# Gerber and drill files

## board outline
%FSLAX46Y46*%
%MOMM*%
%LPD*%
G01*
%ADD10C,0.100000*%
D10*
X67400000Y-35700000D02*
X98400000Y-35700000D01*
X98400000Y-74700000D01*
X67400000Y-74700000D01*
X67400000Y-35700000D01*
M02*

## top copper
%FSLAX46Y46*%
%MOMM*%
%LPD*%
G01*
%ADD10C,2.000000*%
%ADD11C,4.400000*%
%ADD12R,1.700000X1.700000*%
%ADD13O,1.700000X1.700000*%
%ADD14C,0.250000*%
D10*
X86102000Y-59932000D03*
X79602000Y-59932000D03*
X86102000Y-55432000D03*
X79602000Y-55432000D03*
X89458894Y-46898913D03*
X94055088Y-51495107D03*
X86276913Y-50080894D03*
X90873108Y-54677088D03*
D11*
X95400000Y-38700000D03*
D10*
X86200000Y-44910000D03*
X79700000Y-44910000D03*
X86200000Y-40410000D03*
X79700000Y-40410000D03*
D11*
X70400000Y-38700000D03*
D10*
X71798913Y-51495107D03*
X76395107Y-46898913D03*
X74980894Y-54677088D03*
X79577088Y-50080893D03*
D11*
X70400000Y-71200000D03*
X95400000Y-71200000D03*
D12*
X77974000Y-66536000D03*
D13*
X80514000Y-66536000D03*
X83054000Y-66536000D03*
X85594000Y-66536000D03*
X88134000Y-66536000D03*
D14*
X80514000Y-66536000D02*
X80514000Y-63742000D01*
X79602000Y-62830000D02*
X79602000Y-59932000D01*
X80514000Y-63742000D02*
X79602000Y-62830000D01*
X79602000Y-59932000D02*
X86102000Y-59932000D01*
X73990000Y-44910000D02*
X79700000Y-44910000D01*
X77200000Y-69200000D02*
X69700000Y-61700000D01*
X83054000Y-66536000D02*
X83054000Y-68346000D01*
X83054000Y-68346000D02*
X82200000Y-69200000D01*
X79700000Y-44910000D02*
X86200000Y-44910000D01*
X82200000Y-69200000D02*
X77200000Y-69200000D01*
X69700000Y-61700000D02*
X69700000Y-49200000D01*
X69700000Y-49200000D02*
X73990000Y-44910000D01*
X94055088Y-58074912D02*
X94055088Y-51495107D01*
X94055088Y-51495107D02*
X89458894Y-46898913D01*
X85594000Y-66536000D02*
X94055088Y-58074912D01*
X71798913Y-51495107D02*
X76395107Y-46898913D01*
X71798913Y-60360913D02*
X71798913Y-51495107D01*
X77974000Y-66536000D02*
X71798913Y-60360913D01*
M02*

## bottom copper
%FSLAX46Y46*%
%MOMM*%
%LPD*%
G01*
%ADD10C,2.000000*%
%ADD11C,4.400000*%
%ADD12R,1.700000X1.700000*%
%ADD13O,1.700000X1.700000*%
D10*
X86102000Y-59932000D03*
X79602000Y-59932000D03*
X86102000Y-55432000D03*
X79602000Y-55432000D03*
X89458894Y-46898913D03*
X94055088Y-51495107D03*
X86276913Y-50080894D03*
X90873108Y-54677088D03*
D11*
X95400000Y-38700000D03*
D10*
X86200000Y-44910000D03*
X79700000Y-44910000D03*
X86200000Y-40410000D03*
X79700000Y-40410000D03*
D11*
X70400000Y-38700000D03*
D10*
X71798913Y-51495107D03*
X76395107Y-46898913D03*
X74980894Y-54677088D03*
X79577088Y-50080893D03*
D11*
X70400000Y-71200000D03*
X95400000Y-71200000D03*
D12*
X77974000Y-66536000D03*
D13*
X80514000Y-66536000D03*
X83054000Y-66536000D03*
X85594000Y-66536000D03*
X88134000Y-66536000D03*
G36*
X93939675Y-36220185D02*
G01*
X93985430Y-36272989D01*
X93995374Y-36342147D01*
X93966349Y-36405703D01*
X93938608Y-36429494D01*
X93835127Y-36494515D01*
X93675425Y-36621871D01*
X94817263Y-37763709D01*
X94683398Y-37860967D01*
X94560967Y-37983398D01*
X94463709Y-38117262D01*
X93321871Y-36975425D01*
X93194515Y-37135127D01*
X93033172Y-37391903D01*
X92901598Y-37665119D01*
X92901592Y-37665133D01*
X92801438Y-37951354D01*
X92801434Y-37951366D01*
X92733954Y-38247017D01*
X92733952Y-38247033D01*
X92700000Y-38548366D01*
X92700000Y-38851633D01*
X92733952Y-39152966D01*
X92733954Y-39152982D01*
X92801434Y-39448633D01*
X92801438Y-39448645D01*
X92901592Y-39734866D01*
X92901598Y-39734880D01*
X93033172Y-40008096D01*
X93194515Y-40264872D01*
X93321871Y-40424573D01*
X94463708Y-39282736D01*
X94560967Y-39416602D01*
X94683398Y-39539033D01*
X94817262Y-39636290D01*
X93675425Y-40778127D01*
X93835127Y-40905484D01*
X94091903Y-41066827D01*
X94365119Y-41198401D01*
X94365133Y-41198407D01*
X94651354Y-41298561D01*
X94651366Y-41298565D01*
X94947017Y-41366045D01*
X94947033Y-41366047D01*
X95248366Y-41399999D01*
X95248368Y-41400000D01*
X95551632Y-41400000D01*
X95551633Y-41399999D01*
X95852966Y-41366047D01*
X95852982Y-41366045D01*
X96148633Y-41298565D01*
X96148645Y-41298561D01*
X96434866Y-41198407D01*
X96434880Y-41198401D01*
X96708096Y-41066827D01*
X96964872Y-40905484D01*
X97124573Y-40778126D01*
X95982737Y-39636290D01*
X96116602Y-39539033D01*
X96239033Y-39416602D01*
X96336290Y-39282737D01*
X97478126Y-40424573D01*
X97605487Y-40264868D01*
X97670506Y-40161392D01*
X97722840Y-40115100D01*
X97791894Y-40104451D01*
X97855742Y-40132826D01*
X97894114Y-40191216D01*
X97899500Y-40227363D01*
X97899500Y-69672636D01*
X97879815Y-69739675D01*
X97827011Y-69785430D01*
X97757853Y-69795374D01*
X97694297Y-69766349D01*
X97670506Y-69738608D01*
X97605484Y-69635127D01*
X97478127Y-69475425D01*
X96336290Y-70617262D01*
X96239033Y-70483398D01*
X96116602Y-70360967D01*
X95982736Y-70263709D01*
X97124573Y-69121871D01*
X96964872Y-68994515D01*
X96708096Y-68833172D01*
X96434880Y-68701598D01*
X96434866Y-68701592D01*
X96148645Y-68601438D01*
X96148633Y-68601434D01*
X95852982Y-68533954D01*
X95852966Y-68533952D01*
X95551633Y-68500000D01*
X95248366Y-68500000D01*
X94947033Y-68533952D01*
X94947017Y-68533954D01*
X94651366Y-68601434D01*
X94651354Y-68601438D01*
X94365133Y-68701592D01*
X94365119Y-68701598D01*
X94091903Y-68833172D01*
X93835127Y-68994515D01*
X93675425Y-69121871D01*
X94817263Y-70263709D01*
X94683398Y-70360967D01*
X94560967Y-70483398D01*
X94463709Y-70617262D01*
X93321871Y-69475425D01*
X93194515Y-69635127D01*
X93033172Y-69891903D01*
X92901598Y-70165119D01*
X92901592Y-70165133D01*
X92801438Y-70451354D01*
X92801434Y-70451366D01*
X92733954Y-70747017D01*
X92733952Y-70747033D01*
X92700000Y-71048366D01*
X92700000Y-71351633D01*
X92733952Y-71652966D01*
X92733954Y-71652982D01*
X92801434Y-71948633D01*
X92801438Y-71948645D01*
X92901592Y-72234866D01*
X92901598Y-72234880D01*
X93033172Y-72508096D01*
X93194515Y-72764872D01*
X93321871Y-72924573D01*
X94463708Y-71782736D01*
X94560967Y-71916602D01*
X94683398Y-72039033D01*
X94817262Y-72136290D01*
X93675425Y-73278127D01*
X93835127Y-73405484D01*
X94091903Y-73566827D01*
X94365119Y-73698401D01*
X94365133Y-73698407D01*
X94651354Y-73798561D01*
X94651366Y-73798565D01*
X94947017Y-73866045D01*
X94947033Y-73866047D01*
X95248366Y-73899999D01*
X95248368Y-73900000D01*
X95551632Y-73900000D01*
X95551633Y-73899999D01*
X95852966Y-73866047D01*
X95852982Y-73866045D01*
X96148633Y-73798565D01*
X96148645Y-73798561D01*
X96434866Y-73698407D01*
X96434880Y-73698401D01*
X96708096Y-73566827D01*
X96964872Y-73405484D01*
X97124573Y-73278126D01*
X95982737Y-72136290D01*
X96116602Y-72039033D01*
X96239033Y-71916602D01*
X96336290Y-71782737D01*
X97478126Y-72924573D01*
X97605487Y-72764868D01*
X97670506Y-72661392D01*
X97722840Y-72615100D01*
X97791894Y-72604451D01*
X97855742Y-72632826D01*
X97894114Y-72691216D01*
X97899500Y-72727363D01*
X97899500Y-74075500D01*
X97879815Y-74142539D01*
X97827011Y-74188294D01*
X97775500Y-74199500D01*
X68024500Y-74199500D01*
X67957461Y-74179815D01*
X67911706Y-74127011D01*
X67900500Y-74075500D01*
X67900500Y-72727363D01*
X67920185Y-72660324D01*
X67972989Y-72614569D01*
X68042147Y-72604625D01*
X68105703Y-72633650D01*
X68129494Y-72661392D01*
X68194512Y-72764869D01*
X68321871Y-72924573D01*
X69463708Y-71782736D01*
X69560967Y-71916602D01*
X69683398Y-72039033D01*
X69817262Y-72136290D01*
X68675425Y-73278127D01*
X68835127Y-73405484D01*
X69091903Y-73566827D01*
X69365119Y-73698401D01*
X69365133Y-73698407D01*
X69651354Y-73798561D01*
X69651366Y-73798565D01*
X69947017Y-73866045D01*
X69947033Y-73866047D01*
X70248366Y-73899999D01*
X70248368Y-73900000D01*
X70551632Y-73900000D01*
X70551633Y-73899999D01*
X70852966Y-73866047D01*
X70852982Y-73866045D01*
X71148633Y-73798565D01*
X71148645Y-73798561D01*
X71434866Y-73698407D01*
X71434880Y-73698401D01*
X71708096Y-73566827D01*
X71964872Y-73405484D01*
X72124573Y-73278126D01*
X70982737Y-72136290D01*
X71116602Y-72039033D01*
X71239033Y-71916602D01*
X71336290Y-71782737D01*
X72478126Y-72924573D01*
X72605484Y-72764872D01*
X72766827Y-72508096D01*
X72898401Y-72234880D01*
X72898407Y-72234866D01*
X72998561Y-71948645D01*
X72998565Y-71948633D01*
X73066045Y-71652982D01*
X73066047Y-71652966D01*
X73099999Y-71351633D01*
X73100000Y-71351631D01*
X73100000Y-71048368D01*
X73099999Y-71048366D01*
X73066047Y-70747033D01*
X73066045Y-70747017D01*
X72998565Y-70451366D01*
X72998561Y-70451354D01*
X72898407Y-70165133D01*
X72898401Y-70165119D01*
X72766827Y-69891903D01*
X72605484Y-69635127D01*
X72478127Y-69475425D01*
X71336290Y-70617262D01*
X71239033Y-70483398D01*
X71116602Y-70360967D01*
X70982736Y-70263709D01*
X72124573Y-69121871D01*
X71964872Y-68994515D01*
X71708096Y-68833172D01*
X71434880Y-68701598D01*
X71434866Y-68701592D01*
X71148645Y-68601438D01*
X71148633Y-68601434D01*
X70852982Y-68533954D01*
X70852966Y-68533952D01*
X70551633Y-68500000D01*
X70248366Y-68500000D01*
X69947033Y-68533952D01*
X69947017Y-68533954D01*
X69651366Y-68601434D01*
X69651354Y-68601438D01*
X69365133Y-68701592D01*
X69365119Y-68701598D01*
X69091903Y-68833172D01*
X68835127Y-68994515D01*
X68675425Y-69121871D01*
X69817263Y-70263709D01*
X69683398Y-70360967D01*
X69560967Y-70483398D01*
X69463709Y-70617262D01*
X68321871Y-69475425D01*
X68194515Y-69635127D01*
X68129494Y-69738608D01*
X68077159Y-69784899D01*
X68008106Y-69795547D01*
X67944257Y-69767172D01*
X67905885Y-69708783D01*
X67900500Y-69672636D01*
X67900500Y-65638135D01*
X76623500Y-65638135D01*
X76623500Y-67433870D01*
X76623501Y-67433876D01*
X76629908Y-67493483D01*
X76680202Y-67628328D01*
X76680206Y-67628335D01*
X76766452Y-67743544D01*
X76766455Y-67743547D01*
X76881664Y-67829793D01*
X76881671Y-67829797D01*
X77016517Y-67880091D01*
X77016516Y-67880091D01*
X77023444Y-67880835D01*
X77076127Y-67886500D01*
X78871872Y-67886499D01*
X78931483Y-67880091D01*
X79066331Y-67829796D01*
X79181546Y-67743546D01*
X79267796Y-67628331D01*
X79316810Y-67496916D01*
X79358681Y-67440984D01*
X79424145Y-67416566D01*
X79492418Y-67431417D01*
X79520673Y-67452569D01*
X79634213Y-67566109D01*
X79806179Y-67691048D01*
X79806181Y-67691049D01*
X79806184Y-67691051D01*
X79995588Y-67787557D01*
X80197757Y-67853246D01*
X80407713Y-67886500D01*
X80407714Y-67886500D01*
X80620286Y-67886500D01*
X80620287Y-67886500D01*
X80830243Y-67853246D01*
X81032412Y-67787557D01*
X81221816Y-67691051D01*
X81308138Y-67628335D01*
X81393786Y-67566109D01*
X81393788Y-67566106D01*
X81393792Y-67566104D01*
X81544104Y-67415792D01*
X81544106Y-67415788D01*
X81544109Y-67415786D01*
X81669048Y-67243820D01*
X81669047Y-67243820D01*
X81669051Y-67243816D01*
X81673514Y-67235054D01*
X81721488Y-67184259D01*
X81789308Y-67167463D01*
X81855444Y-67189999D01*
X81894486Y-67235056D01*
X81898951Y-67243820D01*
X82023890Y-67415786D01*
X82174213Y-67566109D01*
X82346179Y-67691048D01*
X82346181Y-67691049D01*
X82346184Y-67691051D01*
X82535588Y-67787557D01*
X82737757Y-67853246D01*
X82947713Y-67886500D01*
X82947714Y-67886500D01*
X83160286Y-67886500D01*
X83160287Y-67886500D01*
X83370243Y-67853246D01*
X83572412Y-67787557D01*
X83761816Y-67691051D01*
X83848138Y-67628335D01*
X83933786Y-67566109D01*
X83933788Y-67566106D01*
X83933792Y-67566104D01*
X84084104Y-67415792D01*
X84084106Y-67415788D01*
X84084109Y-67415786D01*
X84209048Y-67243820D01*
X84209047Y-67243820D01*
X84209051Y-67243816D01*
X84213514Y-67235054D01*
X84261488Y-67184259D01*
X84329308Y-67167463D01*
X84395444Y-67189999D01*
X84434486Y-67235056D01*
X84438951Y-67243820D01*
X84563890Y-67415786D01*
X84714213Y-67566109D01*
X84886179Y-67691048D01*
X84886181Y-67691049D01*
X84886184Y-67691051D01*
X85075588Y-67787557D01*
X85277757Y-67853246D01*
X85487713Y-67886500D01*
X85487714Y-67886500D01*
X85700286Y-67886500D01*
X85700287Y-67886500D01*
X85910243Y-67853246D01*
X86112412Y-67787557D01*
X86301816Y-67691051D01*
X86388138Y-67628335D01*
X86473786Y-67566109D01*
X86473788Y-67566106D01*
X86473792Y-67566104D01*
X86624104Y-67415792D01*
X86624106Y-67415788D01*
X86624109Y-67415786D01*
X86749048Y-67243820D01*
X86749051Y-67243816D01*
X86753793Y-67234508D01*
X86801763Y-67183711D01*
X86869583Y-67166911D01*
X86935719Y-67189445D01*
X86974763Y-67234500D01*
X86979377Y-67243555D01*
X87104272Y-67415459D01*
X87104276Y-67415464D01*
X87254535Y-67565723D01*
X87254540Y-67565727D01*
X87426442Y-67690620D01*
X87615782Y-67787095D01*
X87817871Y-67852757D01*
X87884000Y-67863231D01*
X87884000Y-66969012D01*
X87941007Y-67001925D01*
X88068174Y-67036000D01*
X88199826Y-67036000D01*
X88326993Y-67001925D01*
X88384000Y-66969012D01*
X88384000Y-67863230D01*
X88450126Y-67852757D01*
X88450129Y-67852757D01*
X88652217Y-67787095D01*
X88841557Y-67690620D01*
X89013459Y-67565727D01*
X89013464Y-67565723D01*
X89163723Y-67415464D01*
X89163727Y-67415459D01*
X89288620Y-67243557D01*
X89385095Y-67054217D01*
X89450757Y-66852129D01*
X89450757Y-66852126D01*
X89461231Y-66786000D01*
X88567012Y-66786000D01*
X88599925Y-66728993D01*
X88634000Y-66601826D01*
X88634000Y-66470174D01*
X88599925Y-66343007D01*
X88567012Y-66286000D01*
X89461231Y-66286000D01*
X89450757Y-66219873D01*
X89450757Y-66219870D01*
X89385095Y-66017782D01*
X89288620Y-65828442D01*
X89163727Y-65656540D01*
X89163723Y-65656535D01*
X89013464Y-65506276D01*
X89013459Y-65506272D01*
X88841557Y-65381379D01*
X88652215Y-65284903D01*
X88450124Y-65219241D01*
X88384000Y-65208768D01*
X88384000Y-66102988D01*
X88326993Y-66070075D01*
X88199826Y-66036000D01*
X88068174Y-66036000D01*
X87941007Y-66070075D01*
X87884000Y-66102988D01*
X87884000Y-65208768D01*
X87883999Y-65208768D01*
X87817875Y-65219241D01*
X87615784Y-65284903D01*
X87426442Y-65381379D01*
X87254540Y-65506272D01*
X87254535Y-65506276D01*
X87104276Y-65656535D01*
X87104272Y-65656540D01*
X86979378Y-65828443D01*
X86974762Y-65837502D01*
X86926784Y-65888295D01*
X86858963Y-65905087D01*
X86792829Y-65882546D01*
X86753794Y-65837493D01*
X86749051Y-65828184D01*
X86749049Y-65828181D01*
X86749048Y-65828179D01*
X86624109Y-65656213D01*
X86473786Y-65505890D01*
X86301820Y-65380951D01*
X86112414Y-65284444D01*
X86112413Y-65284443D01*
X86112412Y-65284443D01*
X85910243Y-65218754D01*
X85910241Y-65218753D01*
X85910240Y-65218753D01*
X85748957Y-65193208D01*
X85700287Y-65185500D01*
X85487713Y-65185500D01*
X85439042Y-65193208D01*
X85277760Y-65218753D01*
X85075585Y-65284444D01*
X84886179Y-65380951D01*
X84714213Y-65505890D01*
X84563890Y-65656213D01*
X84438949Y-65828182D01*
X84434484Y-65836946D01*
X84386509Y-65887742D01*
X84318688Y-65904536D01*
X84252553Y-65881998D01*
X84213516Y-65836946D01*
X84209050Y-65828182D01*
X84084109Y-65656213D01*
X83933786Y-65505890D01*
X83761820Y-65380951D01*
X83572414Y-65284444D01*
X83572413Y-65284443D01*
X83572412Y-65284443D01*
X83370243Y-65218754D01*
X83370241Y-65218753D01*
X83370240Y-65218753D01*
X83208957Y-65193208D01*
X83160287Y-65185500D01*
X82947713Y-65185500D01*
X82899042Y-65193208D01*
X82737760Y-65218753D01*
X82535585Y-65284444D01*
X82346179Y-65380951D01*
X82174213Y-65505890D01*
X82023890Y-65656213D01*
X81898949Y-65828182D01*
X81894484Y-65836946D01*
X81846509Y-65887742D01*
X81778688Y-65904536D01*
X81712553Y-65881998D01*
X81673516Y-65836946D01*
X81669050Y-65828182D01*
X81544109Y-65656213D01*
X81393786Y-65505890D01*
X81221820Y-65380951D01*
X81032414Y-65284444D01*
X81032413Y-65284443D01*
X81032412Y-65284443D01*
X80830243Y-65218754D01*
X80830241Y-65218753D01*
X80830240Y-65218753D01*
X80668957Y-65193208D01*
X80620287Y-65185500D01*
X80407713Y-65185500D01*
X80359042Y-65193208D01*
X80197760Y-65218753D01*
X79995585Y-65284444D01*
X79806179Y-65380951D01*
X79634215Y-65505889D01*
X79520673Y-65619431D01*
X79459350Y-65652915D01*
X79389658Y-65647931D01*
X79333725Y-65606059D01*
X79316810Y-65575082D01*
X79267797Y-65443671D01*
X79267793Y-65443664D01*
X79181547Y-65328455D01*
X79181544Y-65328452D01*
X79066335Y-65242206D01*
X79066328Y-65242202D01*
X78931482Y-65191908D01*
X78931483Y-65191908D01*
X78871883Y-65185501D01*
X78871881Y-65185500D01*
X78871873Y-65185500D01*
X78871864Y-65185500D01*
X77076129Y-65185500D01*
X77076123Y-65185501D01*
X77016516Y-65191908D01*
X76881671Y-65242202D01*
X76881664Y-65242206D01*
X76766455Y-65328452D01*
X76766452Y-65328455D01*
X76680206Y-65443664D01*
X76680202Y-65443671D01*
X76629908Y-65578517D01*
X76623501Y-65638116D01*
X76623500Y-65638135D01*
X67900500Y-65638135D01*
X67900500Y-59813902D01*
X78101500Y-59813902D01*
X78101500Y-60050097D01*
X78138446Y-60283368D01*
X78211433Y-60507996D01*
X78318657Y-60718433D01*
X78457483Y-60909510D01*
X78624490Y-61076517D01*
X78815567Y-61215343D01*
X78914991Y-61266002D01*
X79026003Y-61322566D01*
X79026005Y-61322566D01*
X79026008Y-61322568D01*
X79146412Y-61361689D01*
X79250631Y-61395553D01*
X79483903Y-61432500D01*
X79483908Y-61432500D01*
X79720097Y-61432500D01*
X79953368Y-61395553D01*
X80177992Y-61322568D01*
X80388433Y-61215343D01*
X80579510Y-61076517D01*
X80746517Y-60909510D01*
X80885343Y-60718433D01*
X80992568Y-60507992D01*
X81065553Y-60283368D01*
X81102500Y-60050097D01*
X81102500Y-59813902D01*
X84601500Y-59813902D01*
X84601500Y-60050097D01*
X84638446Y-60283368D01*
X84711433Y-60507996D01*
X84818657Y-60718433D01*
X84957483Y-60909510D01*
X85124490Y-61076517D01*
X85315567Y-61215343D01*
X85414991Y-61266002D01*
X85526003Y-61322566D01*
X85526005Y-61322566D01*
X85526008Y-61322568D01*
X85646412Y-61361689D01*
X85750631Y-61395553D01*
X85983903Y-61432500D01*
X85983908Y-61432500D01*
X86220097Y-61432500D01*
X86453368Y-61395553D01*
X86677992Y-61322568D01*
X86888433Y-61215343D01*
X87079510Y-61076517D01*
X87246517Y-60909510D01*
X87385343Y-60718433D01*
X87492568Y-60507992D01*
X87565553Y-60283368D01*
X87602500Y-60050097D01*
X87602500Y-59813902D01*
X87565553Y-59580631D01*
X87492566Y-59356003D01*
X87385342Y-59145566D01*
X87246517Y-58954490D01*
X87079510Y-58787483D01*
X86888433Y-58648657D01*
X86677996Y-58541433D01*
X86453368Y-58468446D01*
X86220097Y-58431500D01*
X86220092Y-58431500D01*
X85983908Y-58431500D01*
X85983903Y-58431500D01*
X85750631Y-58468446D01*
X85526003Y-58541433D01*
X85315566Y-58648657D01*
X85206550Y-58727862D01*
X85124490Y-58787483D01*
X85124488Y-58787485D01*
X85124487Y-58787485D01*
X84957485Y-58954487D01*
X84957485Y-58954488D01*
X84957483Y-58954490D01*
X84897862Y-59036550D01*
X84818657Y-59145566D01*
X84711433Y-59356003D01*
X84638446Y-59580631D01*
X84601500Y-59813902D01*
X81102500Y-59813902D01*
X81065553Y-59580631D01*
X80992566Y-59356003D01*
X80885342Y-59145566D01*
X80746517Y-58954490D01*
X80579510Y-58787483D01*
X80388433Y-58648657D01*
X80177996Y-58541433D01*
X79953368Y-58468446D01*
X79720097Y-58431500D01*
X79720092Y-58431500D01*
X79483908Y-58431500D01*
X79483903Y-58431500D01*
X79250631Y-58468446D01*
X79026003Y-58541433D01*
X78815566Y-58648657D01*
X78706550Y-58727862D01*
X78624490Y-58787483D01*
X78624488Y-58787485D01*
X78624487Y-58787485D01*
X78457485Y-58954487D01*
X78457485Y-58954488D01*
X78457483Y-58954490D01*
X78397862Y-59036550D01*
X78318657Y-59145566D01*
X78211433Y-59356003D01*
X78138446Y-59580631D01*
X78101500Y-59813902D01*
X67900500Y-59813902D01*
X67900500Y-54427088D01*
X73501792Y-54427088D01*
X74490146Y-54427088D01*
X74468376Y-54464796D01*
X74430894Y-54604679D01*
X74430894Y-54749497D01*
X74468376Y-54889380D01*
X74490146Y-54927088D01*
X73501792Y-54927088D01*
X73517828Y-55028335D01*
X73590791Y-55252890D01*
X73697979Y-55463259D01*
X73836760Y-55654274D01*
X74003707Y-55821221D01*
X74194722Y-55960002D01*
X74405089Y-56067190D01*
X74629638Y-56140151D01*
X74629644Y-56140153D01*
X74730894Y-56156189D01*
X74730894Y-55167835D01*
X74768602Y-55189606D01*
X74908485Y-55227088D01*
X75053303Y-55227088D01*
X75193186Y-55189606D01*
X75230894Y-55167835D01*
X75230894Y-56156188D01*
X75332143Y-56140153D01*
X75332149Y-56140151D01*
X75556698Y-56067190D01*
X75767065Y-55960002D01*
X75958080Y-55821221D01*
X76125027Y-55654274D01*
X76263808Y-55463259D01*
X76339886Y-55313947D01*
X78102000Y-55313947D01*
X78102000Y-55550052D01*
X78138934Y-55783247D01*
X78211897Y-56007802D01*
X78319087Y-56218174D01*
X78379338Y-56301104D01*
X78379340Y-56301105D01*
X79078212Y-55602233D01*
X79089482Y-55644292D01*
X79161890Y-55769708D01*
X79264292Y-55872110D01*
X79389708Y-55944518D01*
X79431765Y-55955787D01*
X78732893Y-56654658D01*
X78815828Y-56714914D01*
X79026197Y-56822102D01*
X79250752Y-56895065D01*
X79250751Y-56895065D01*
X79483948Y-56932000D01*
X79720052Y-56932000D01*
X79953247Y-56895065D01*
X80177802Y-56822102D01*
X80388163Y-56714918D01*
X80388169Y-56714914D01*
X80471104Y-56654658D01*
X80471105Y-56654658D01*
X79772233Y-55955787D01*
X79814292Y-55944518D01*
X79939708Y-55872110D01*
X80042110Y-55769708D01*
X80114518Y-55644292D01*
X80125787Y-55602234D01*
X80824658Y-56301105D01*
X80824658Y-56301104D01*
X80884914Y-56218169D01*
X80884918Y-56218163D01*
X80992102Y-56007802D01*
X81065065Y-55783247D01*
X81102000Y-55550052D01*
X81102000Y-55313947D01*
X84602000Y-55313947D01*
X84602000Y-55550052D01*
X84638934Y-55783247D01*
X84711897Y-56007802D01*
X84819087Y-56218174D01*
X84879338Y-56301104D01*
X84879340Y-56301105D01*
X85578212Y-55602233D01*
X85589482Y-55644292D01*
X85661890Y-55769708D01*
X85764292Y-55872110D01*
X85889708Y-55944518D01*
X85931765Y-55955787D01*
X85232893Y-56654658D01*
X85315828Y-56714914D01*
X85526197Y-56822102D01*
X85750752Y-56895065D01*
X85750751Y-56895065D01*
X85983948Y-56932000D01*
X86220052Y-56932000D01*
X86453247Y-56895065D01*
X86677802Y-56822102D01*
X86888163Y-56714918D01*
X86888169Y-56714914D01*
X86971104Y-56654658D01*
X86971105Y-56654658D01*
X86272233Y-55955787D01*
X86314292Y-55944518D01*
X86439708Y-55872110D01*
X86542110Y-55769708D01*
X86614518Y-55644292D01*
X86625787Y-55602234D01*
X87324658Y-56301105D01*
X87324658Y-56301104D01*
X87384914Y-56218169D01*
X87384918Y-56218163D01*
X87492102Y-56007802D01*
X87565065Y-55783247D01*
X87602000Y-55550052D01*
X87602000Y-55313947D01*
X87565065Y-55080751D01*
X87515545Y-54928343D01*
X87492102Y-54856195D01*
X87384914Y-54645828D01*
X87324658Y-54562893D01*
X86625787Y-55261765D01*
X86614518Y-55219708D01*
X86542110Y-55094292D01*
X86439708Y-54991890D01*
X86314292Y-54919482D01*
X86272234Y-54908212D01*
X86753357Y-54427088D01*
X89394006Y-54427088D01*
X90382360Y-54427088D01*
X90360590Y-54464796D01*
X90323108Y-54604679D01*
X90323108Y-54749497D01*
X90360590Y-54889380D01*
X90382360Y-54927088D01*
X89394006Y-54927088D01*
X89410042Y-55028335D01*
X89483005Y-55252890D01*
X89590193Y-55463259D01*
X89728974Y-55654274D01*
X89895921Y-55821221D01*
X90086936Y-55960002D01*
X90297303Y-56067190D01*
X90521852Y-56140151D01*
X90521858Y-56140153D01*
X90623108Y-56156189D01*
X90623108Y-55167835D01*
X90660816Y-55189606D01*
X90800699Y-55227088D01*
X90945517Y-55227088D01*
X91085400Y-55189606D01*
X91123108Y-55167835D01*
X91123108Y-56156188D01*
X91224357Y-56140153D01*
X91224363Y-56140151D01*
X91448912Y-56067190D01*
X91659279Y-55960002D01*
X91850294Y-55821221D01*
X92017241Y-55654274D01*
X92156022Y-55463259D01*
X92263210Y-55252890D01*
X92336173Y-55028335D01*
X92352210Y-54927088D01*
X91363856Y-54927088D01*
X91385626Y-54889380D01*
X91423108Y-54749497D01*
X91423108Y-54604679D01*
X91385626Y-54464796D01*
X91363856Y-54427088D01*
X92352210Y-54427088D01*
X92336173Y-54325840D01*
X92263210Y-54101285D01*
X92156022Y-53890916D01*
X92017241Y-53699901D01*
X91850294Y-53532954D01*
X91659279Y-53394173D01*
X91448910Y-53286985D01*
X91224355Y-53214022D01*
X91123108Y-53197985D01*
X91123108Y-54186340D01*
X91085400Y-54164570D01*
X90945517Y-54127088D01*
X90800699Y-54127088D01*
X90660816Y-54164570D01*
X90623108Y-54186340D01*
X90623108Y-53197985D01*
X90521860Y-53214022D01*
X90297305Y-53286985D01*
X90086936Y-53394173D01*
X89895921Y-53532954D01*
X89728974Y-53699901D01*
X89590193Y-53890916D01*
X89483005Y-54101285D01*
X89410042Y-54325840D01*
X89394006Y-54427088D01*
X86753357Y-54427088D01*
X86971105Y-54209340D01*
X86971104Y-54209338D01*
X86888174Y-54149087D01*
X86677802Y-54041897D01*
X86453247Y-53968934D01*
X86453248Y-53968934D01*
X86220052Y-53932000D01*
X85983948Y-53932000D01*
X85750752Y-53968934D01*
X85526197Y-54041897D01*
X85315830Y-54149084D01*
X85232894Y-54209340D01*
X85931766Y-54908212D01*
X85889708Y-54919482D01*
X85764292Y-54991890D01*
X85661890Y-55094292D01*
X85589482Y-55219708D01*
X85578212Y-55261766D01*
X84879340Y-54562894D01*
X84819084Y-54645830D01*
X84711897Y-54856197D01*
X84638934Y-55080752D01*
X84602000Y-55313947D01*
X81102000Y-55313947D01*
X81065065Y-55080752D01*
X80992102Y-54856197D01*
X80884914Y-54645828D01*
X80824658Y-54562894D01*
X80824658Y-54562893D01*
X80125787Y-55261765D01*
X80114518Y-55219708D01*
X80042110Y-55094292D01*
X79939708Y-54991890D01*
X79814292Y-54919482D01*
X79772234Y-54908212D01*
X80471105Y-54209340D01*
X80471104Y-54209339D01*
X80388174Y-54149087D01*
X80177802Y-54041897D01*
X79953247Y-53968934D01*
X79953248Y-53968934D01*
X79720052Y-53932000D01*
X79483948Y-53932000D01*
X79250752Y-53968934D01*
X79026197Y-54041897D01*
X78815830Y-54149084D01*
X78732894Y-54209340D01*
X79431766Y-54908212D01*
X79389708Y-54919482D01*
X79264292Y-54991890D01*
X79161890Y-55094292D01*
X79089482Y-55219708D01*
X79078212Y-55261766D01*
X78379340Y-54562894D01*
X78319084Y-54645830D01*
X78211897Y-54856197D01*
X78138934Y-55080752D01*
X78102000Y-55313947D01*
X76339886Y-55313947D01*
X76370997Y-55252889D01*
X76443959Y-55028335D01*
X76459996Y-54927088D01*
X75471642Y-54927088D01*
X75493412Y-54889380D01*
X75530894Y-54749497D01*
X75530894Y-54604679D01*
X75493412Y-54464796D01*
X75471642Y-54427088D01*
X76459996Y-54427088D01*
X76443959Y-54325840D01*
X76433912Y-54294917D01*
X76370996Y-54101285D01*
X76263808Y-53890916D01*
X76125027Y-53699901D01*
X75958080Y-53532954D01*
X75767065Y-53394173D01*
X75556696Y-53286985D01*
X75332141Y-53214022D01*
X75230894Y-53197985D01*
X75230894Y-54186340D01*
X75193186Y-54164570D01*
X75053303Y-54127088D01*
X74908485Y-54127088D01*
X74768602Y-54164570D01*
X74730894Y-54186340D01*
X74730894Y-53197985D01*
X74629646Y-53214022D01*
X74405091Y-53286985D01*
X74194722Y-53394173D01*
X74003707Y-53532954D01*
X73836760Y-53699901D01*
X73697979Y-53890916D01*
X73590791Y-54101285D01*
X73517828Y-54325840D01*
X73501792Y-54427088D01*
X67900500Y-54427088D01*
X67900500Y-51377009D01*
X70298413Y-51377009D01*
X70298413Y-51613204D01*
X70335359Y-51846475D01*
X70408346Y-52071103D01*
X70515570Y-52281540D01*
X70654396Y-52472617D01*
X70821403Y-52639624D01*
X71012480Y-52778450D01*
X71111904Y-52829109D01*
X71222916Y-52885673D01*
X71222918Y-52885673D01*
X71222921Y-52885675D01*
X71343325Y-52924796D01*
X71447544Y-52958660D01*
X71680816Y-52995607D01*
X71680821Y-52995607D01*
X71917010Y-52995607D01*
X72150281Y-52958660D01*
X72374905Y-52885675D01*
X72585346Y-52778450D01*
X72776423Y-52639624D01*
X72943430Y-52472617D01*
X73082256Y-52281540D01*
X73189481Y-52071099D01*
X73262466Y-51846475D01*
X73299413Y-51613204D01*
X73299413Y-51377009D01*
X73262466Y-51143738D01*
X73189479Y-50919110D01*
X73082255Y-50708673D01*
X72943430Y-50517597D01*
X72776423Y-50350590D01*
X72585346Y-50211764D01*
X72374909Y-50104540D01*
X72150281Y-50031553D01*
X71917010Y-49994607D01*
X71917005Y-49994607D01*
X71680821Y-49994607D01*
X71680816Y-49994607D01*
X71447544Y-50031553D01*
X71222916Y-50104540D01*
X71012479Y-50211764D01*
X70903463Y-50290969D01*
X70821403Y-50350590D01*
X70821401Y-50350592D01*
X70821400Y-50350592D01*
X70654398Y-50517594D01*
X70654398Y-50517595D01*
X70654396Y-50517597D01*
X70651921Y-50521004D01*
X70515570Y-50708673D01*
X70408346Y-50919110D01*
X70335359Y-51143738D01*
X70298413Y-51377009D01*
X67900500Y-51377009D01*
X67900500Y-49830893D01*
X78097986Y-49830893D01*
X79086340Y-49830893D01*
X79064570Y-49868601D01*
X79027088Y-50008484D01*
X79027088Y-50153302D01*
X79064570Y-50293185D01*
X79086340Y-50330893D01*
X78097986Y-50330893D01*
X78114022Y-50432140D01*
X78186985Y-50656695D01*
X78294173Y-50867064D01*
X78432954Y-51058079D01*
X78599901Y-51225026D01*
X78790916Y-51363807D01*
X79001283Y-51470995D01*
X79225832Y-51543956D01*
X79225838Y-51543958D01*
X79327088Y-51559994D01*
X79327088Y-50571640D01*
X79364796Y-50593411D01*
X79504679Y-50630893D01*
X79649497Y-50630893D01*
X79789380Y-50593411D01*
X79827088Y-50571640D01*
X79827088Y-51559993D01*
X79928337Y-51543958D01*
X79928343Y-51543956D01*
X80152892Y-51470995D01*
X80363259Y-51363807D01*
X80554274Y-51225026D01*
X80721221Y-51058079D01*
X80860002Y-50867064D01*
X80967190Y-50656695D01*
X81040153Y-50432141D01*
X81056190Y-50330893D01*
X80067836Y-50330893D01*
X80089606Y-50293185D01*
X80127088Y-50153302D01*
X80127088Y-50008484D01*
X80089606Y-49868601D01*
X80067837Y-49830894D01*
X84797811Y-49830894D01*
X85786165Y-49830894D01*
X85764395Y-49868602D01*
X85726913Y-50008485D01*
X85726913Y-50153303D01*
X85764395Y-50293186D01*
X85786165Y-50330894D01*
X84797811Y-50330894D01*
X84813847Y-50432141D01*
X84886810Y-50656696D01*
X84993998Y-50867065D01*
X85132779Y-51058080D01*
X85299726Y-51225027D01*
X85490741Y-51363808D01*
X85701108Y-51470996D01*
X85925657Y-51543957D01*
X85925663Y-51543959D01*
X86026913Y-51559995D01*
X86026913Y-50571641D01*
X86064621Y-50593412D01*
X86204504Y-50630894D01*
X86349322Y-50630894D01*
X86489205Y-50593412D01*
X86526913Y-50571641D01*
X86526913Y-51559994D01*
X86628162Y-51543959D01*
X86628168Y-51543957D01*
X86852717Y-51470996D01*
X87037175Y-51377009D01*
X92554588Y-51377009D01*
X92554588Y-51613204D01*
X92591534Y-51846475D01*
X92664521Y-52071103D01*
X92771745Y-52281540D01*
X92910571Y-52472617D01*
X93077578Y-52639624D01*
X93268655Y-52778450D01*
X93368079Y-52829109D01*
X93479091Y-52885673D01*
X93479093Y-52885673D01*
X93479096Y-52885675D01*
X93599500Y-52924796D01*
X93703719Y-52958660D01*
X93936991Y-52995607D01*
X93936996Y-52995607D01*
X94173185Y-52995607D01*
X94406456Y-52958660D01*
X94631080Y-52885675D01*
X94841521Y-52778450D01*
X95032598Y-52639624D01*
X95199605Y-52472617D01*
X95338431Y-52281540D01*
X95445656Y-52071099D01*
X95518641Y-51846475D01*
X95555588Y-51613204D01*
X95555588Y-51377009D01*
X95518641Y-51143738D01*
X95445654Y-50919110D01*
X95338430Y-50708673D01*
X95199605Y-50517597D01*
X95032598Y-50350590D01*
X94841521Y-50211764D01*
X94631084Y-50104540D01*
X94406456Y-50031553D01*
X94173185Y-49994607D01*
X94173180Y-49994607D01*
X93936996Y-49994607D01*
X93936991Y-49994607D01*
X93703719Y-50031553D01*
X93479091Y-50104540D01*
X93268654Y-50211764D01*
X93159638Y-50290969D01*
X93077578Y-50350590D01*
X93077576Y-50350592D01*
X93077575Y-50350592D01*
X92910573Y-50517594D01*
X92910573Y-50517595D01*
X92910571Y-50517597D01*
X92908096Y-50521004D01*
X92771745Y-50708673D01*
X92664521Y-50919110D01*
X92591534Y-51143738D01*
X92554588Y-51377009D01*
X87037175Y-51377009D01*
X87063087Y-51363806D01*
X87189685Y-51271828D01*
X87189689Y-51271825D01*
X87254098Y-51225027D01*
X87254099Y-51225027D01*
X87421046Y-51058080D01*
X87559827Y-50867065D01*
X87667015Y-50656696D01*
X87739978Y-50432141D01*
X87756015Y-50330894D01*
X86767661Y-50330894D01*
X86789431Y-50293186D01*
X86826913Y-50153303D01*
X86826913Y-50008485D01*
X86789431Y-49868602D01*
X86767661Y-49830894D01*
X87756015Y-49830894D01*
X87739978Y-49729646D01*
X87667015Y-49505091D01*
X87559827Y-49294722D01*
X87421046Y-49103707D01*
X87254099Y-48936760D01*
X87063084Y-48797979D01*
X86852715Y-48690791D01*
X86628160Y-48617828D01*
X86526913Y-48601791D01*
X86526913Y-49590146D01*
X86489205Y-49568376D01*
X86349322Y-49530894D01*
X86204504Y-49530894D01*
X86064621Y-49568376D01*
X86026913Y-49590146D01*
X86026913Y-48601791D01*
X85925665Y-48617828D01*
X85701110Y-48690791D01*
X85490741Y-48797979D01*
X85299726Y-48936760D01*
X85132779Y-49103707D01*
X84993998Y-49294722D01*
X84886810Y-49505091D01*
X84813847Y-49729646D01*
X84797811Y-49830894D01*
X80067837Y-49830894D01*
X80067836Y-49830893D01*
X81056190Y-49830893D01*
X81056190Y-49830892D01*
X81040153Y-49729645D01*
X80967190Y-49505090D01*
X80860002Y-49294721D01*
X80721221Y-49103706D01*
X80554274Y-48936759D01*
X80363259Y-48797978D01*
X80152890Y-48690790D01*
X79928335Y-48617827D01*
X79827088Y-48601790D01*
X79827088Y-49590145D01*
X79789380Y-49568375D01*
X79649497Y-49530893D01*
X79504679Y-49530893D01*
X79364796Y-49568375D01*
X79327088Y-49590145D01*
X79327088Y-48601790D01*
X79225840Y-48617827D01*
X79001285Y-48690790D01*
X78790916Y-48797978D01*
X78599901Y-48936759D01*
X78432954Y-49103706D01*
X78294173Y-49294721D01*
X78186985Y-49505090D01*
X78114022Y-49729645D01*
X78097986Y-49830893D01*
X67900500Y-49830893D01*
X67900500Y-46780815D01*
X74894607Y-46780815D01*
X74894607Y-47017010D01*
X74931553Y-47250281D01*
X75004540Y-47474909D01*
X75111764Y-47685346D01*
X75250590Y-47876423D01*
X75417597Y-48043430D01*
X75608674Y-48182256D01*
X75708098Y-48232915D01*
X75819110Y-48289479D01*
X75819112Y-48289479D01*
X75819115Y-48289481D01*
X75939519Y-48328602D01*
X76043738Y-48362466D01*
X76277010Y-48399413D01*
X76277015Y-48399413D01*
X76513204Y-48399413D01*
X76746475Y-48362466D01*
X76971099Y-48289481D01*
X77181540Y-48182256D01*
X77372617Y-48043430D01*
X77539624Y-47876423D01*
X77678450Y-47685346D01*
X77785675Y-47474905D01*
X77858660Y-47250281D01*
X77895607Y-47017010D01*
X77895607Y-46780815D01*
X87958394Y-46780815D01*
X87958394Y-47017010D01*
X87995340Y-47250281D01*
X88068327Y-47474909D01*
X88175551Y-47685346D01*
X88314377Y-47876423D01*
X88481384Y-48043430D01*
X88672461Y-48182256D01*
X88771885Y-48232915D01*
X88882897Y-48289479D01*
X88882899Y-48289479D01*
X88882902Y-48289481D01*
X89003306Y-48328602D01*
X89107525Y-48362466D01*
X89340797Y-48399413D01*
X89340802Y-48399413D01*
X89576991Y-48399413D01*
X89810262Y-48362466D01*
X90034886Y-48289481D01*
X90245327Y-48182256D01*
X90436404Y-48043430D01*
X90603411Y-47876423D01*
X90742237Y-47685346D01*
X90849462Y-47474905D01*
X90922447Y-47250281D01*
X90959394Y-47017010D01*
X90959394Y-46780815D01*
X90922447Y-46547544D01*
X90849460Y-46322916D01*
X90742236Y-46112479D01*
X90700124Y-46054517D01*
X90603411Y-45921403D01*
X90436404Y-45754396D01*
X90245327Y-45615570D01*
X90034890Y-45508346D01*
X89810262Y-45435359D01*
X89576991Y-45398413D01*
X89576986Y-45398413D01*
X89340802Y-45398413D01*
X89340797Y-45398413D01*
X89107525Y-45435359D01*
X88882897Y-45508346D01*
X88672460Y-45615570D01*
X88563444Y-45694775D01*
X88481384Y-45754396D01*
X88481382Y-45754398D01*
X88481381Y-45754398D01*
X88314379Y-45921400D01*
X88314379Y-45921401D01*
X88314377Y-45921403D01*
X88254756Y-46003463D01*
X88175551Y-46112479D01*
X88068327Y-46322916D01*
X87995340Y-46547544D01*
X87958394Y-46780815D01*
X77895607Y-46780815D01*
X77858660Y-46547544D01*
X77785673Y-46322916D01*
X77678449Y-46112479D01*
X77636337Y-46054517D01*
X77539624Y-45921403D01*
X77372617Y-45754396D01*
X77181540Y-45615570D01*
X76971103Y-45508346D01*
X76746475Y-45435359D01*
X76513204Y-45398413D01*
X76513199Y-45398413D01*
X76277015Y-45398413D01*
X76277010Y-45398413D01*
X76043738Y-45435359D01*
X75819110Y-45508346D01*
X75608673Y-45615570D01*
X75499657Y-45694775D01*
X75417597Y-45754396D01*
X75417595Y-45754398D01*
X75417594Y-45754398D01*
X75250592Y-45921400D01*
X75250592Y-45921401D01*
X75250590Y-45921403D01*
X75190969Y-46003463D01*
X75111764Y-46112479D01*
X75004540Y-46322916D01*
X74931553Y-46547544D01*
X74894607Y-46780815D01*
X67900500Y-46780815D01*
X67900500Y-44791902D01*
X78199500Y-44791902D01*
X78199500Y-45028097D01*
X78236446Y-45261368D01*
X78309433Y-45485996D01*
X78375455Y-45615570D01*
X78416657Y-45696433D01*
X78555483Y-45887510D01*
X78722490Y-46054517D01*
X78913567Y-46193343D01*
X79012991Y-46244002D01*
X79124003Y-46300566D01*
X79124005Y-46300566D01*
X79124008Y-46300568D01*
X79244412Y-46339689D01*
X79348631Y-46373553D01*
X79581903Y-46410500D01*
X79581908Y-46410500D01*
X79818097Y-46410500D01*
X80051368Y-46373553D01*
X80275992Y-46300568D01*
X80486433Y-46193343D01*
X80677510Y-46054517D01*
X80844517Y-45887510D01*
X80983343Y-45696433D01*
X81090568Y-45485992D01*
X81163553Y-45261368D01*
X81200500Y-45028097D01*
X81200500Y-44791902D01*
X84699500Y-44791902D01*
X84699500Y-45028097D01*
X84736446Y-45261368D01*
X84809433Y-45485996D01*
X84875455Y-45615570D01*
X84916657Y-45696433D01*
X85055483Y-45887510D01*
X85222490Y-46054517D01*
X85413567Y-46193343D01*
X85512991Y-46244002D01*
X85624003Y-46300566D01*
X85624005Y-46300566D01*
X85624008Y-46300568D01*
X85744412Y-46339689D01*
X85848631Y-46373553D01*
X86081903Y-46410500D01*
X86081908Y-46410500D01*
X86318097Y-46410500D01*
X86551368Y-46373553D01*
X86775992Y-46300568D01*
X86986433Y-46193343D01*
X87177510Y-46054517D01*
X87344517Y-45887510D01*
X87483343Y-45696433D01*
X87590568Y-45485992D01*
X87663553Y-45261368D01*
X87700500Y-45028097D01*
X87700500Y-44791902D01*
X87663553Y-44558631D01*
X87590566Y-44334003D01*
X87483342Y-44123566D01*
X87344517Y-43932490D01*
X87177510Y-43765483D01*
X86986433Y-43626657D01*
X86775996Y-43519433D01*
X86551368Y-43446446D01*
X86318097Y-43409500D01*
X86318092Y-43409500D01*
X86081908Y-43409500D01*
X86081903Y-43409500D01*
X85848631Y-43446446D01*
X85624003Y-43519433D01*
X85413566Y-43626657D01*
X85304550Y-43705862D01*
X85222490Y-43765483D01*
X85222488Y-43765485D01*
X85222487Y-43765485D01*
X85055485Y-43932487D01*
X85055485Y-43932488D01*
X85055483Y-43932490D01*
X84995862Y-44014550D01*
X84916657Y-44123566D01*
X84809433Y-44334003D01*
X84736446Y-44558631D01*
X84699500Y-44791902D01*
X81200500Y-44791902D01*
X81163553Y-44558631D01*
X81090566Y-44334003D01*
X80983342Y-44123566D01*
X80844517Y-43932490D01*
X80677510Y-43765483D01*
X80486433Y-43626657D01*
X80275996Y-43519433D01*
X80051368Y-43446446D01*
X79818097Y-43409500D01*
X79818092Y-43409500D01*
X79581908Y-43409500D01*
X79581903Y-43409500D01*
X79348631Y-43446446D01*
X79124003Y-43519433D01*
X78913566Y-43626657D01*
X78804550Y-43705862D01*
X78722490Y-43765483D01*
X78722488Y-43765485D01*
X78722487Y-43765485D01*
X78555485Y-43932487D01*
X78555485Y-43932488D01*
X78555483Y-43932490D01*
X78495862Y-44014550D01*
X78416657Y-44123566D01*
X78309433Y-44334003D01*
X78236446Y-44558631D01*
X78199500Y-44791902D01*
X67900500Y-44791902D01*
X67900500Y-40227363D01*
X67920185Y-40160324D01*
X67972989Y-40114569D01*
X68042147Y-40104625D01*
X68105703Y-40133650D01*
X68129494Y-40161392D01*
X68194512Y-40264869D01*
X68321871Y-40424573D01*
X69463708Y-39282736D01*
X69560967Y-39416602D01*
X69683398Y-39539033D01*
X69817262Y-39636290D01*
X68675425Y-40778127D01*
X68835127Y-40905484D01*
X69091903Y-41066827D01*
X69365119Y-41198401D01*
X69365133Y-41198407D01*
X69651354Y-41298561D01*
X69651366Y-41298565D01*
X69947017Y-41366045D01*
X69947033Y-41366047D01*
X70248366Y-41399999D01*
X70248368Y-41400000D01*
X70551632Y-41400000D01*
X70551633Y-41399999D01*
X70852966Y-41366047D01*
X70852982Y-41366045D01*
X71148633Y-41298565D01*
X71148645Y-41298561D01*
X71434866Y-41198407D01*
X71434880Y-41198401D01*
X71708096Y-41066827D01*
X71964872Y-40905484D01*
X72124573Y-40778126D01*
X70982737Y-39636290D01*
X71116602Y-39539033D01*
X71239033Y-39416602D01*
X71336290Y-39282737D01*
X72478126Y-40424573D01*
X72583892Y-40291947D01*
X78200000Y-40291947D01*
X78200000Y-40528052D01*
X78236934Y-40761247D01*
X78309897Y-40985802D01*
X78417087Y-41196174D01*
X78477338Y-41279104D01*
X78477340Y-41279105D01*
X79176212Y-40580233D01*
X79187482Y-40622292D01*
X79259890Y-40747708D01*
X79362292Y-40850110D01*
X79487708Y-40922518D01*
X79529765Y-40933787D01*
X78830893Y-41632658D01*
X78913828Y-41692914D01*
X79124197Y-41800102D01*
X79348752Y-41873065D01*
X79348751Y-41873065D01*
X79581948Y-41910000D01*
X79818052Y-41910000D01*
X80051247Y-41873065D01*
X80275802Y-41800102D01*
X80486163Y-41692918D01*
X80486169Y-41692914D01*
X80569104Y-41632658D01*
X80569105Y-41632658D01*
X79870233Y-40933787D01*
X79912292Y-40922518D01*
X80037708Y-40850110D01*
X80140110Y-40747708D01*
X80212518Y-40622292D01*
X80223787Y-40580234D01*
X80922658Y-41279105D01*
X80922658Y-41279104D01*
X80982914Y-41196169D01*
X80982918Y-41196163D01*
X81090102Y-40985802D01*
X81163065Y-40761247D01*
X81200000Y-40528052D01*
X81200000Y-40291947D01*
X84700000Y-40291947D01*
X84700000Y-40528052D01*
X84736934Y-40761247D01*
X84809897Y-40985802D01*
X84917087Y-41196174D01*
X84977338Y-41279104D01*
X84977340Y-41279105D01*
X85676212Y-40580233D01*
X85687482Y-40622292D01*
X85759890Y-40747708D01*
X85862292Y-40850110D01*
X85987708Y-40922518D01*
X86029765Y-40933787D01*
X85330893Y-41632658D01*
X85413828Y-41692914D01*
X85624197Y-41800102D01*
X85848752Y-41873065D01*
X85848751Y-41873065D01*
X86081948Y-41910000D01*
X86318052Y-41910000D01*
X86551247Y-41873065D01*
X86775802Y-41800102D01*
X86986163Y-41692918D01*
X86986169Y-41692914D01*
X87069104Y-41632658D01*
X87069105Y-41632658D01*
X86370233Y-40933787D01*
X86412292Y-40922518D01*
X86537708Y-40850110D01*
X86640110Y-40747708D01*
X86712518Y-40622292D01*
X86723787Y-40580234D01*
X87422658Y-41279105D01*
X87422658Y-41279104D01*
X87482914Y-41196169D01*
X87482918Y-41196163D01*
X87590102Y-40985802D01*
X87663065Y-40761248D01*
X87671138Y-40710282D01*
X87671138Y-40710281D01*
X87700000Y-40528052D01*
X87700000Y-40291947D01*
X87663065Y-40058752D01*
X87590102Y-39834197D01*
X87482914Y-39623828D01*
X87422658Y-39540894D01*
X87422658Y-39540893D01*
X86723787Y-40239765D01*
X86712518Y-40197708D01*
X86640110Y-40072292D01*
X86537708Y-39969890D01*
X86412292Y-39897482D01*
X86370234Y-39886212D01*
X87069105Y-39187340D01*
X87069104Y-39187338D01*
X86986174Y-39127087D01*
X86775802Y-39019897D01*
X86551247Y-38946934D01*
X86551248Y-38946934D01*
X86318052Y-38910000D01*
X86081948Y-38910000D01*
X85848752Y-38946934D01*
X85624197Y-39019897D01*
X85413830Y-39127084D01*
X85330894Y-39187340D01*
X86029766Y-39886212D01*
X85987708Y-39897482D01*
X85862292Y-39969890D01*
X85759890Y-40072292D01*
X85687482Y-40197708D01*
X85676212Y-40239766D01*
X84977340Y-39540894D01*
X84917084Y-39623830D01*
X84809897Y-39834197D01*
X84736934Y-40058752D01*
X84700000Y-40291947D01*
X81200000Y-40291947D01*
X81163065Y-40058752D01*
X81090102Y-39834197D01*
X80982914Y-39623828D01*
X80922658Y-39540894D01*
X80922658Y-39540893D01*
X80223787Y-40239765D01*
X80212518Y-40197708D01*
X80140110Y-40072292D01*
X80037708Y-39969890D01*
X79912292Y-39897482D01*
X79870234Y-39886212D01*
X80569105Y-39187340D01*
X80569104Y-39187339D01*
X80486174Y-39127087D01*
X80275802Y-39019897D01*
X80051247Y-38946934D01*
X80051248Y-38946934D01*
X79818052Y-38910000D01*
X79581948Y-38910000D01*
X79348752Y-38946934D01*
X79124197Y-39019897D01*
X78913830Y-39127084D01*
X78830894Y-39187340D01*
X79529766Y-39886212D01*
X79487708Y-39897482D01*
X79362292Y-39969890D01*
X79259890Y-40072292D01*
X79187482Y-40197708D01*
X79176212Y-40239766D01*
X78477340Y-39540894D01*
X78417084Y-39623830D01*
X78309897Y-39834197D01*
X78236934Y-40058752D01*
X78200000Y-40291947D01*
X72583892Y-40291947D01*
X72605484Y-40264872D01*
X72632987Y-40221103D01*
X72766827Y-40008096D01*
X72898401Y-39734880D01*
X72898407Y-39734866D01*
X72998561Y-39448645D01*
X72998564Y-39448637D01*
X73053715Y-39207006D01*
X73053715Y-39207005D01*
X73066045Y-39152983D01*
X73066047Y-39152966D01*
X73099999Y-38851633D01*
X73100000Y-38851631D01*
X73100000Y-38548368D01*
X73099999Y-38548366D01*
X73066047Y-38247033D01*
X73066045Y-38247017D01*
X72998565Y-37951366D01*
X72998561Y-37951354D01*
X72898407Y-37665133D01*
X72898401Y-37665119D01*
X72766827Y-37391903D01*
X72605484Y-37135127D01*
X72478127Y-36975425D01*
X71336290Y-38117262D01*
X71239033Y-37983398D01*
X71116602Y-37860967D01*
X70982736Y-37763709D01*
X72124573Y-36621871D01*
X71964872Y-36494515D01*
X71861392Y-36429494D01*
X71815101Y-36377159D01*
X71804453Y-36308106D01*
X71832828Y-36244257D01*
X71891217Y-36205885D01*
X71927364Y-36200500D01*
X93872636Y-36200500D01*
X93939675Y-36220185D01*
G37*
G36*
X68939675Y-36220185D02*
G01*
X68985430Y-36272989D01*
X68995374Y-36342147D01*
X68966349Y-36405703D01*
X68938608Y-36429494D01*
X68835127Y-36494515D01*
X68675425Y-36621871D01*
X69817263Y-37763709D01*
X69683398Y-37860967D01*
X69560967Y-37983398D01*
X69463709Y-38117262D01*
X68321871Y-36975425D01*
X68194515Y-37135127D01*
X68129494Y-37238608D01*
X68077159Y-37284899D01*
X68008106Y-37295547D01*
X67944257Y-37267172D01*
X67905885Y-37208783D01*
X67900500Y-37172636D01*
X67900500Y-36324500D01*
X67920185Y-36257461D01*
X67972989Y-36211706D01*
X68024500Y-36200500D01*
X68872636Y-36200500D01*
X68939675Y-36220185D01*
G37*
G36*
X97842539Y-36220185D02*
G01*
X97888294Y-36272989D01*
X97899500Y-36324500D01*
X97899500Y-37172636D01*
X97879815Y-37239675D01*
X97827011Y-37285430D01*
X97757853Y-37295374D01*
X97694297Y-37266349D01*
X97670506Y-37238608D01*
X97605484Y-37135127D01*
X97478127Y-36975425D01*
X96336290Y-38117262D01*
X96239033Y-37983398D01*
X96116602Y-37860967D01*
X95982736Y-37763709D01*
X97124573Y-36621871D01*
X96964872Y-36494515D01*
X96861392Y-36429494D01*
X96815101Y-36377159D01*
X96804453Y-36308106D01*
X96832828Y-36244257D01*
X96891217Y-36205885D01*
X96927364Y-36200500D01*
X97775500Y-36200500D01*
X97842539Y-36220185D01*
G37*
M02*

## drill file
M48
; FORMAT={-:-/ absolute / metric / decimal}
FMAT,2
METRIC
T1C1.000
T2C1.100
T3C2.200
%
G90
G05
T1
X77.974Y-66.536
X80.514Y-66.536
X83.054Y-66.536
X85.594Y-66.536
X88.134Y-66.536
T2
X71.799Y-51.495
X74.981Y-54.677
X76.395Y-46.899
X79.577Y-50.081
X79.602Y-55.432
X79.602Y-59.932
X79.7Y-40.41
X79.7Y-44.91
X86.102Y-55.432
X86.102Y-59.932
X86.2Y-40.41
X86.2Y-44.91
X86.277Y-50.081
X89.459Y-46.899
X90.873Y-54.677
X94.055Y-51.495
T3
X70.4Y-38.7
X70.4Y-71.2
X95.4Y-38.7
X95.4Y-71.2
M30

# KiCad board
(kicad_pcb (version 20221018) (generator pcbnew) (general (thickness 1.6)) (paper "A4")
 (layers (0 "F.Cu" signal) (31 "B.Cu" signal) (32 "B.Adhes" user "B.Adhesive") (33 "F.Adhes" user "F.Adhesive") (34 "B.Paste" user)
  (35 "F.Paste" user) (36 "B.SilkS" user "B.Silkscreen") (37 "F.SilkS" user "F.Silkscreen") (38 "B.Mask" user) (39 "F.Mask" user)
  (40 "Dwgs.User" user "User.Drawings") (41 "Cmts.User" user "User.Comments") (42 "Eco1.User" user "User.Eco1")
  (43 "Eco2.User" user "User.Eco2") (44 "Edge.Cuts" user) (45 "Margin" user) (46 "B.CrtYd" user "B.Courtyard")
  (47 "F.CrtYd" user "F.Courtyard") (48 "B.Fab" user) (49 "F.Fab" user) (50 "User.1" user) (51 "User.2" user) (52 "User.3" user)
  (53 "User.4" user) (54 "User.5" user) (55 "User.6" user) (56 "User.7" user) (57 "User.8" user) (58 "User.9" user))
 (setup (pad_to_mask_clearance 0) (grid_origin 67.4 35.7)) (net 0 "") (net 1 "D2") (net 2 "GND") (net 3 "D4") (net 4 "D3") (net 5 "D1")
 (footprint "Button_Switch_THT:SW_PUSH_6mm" (layer "F.Cu") (at 86.102 59.932 180)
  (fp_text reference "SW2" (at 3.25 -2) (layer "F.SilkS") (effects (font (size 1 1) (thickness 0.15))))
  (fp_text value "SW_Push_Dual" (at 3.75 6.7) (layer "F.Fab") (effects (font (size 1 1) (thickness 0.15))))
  (pad "1" thru_hole circle (at 0 0 270) (size 2 2) (drill 1.1) (layers "*.Cu" "*.Mask") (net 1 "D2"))
  (pad "1" thru_hole circle (at 6.5 0 270) (size 2 2) (drill 1.1) (layers "*.Cu" "*.Mask") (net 1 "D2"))
  (pad "2" thru_hole circle (at 0 4.5 270) (size 2 2) (drill 1.1) (layers "*.Cu" "*.Mask") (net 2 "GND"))
  (pad "2" thru_hole circle (at 6.5 4.5 270) (size 2 2) (drill 1.1) (layers "*.Cu" "*.Mask") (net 2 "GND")))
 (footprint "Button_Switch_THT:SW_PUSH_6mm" (layer "F.Cu") (at 89.458894 46.898913 -45)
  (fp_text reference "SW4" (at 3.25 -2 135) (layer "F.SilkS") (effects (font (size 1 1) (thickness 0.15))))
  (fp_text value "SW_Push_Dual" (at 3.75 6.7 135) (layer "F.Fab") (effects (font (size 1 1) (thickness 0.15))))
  (pad "1" thru_hole circle (at 0 0 45) (size 2 2) (drill 1.1) (layers "*.Cu" "*.Mask") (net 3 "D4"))
  (pad "1" thru_hole circle (at 6.5 0 45) (size 2 2) (drill 1.1) (layers "*.Cu" "*.Mask") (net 3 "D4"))
  (pad "2" thru_hole circle (at 0 4.5 45) (size 2 2) (drill 1.1) (layers "*.Cu" "*.Mask") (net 2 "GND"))
  (pad "2" thru_hole circle (at 6.5 4.5 45) (size 2 2) (drill 1.1) (layers "*.Cu" "*.Mask") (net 2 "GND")))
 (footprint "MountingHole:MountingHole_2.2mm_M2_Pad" (layer "F.Cu") (at 95.4 38.7 90)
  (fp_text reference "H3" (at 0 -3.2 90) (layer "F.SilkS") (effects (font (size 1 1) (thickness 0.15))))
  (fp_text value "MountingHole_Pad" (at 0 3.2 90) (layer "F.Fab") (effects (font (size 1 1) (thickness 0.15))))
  (pad "1" thru_hole circle (at 0 0 90) (size 4.4 4.4) (drill 2.2) (layers "*.Cu" "*.Mask") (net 2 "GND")))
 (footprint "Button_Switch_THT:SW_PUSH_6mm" (layer "F.Cu") (at 86.2 44.91 180)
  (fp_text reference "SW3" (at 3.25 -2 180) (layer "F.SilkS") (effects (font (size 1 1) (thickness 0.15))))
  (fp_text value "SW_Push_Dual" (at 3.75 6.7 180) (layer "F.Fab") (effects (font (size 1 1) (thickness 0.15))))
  (pad "1" thru_hole circle (at 0 0 270) (size 2 2) (drill 1.1) (layers "*.Cu" "*.Mask") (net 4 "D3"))
  (pad "1" thru_hole circle (at 6.5 0 270) (size 2 2) (drill 1.1) (layers "*.Cu" "*.Mask") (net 4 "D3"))
  (pad "2" thru_hole circle (at 0 4.5 270) (size 2 2) (drill 1.1) (layers "*.Cu" "*.Mask") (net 2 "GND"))
  (pad "2" thru_hole circle (at 6.5 4.5 270) (size 2 2) (drill 1.1) (layers "*.Cu" "*.Mask") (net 2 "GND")))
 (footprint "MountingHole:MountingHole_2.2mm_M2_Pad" (layer "F.Cu") (at 70.4 38.7 -90)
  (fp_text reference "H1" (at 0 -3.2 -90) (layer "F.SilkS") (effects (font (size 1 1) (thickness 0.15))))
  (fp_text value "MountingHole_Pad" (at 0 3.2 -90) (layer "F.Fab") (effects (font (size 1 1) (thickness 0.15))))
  (pad "1" thru_hole circle (at 0 0 270) (size 4.4 4.4) (drill 2.2) (layers "*.Cu" "*.Mask") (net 2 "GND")))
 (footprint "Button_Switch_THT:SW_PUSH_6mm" (layer "F.Cu") (at 71.798913 51.495107 45)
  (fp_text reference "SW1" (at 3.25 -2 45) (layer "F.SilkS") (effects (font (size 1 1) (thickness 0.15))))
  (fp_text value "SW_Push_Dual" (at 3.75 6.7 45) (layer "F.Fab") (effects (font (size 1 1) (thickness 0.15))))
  (pad "1" thru_hole circle (at 0 0 135) (size 2 2) (drill 1.1) (layers "*.Cu" "*.Mask") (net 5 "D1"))
  (pad "1" thru_hole circle (at 6.5 0 135) (size 2 2) (drill 1.1) (layers "*.Cu" "*.Mask") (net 5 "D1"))
  (pad "2" thru_hole circle (at 0 4.5 135) (size 2 2) (drill 1.1) (layers "*.Cu" "*.Mask") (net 2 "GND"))
  (pad "2" thru_hole circle (at 6.5 4.5 135) (size 2 2) (drill 1.1) (layers "*.Cu" "*.Mask") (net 2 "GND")))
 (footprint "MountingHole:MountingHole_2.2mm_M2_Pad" (layer "F.Cu") (at 70.4 71.2 -90)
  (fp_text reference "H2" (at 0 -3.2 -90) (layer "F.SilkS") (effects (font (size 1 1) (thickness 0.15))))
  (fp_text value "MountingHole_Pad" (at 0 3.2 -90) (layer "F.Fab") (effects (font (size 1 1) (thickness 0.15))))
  (pad "1" thru_hole circle (at 0 0 270) (size 4.4 4.4) (drill 2.2) (layers "*.Cu" "*.Mask") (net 2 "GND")))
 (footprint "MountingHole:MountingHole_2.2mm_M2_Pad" (layer "F.Cu") (at 95.4 71.2 90)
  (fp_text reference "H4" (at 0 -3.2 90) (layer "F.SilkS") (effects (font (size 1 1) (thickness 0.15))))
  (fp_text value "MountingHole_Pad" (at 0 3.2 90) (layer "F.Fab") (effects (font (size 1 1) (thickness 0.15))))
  (pad "1" thru_hole circle (at 0 0 90) (size 4.4 4.4) (drill 2.2) (layers "*.Cu" "*.Mask") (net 2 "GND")))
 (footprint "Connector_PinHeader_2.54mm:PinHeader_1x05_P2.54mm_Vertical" (layer "B.Cu") (at 77.974 66.536 -90)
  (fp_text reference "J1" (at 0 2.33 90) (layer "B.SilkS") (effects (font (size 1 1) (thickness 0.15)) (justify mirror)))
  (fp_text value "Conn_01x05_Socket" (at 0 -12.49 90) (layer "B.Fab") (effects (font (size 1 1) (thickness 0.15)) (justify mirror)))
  (pad "1" thru_hole rect (at 0 0 270) (size 1.7 1.7) (drill 1) (layers "*.Cu" "*.Mask") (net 5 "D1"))
  (pad "2" thru_hole oval (at 0 -2.54 270) (size 1.7 1.7) (drill 1) (layers "*.Cu" "*.Mask") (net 1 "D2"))
  (pad "3" thru_hole oval (at 0 -5.08 270) (size 1.7 1.7) (drill 1) (layers "*.Cu" "*.Mask") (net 4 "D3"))
  (pad "4" thru_hole oval (at 0 -7.62 270) (size 1.7 1.7) (drill 1) (layers "*.Cu" "*.Mask") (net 3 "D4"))
  (pad "5" thru_hole oval (at 0 -10.16 270) (size 1.7 1.7) (drill 1) (layers "*.Cu" "*.Mask") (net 2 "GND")))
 (gr_rect (start 67.4 35.7) (end 98.4 74.7) (stroke (width 0.1) (type default)) (fill none) (layer "Edge.Cuts"))
 (segment (start 80.514 66.536) (end 80.514 63.742) (width 0.25) (layer "F.Cu") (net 1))
 (segment (start 79.602 62.83) (end 79.602 59.932) (width 0.25) (layer "F.Cu") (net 1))
 (segment (start 80.514 63.742) (end 79.602 62.83) (width 0.25) (layer "F.Cu") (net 1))
 (segment (start 79.602 59.932) (end 86.102 59.932) (width 0.25) (layer "F.Cu") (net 1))
 (segment (start 73.99 44.91) (end 79.7 44.91) (width 0.25) (layer "F.Cu") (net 4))
 (segment (start 77.2 69.2) (end 69.7 61.7) (width 0.25) (layer "F.Cu") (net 4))
 (segment (start 83.054 66.536) (end 83.054 68.346) (width 0.25) (layer "F.Cu") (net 4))
 (segment (start 83.054 68.346) (end 82.2 69.2) (width 0.25) (layer "F.Cu") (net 4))
 (segment (start 79.7 44.91) (end 86.2 44.91) (width 0.25) (layer "F.Cu") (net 4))
 (segment (start 82.2 69.2) (end 77.2 69.2) (width 0.25) (layer "F.Cu") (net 4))
 (segment (start 69.7 61.7) (end 69.7 49.2) (width 0.25) (layer "F.Cu") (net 4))
 (segment (start 69.7 49.2) (end 73.99 44.91) (width 0.25) (layer "F.Cu") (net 4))
 (segment (start 94.055088 58.074912) (end 94.055088 51.495107) (width 0.25) (layer "F.Cu") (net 3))
 (segment (start 94.055088 51.495107) (end 89.458894 46.898913) (width 0.25) (layer "F.Cu") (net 3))
 (segment (start 85.594 66.536) (end 94.055088 58.074912) (width 0.25) (layer "F.Cu") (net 3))
 (segment (start 71.798913 51.495107) (end 76.395107 46.898913) (width 0.25) (layer "F.Cu") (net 5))
 (segment (start 71.798913 60.360913) (end 71.798913 51.495107) (width 0.25) (layer "F.Cu") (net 5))
 (segment (start 77.974 66.536) (end 71.798913 60.360913) (width 0.25) (layer "F.Cu") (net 5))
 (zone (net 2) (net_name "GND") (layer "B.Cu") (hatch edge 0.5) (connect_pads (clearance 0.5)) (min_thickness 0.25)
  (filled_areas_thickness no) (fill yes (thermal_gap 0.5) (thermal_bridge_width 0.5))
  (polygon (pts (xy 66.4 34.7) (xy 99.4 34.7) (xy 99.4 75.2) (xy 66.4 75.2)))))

